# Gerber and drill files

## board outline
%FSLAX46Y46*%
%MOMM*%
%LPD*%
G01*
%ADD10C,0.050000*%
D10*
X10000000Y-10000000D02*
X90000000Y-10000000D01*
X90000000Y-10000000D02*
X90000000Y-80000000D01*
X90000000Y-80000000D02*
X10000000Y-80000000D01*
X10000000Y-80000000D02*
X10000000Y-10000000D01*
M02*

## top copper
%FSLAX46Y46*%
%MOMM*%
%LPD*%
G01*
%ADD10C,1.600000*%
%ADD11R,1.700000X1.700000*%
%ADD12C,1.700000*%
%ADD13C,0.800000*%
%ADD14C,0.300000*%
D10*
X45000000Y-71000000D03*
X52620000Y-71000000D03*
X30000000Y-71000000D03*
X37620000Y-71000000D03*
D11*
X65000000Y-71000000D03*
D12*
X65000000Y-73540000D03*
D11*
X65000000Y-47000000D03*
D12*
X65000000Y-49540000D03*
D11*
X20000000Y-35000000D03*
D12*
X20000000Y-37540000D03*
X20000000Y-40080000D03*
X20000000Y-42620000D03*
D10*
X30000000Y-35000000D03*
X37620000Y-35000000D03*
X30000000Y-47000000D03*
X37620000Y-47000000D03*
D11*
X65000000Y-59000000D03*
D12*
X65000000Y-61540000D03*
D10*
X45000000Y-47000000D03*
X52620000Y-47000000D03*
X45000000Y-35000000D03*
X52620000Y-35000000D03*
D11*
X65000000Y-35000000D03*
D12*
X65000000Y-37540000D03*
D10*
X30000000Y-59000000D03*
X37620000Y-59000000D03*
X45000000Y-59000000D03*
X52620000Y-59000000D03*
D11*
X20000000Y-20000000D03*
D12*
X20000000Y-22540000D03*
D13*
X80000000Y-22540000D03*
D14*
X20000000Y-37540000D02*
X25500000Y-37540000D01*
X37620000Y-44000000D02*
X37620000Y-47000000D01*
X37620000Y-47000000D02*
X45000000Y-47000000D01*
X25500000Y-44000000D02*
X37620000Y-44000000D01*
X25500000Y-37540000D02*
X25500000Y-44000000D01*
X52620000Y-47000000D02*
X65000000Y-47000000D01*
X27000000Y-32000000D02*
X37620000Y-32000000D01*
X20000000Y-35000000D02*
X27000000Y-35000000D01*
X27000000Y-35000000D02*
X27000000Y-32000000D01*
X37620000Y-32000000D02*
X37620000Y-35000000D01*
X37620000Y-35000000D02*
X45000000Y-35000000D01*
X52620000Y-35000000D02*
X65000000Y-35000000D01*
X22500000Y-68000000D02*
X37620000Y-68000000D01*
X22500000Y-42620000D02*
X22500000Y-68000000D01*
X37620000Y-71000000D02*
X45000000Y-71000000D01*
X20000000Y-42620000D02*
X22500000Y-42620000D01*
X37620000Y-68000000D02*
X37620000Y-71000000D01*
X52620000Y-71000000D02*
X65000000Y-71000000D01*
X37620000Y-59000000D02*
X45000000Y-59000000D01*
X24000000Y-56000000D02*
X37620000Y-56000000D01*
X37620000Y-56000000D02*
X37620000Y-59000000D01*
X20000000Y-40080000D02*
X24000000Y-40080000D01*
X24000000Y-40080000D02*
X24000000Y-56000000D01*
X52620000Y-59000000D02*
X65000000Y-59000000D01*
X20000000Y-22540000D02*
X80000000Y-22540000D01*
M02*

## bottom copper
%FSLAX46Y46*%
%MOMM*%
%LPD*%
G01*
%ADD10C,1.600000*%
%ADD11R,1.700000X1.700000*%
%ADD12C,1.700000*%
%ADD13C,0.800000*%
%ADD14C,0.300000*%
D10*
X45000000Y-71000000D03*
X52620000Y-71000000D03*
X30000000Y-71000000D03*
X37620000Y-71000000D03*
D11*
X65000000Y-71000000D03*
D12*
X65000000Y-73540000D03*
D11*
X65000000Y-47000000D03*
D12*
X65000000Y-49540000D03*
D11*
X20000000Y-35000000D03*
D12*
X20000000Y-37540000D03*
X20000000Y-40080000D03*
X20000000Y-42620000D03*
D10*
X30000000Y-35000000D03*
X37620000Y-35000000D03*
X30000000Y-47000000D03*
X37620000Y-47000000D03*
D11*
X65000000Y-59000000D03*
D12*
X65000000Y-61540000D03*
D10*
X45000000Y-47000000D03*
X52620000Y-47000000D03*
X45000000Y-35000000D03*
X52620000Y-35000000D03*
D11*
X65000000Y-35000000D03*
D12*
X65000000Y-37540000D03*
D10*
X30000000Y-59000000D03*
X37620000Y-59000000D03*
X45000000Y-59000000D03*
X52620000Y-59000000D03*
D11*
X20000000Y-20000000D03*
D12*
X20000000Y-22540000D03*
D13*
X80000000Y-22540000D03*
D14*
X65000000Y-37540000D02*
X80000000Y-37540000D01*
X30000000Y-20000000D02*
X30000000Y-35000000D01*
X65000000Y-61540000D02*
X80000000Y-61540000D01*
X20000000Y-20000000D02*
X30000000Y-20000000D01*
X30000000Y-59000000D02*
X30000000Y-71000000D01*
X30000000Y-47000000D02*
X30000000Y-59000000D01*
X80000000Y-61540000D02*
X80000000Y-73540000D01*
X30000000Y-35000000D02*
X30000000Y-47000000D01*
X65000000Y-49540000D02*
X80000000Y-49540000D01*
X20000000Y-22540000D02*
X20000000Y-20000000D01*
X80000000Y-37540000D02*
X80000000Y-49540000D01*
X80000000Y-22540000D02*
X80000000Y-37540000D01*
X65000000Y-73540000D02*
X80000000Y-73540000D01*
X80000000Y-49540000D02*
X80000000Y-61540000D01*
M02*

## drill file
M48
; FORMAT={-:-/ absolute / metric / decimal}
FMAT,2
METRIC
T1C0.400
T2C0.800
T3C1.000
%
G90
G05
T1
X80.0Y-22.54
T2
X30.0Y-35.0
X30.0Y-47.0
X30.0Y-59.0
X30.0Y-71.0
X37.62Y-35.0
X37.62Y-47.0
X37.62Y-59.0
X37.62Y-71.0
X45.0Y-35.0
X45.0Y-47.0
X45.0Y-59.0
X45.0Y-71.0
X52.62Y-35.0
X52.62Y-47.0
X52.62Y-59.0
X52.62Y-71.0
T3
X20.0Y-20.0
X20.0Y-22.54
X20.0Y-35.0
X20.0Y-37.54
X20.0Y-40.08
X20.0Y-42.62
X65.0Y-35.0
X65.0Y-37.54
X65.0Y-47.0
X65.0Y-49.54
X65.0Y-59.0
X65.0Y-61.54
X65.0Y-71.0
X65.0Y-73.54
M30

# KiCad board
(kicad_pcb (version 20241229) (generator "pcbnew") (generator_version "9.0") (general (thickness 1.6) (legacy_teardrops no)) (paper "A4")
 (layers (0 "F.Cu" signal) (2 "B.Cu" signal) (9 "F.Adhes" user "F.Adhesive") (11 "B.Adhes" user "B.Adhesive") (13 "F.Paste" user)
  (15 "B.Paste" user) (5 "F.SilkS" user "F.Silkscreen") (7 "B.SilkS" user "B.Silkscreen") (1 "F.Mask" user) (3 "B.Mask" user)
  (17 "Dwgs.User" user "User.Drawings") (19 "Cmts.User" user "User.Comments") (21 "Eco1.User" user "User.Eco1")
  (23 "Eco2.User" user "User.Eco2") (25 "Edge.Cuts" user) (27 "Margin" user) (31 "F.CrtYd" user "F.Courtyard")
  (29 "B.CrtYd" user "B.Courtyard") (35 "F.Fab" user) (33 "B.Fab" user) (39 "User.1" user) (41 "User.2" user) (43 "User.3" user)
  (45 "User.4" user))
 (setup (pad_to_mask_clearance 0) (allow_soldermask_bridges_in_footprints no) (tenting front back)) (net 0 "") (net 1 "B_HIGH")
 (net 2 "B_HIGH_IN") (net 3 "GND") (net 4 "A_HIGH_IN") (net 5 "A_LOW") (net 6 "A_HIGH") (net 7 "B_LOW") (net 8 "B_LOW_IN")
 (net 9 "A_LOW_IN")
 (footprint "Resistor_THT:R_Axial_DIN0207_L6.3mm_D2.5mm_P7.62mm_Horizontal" (layer "F.Cu") (at 45 71)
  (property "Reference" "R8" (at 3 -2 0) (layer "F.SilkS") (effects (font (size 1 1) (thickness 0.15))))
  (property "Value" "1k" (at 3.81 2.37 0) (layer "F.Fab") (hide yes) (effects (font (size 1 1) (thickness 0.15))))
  (pad "1" thru_hole circle (at 0 0) (size 1.6 1.6) (drill 0.8) (layers "*.Cu" "*.Mask") (remove_unused_layers no) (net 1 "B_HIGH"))
  (pad "2" thru_hole circle (at 7.62 0) (size 1.6 1.6) (drill 0.8) (layers "*.Cu" "*.Mask") (remove_unused_layers no) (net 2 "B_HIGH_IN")))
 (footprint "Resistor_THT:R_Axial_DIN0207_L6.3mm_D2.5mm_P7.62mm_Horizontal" (layer "F.Cu") (at 30 71)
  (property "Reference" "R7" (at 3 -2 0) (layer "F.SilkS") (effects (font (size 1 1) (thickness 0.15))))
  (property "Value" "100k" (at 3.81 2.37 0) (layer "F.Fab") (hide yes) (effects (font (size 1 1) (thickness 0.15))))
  (pad "1" thru_hole circle (at 0 0) (size 1.6 1.6) (drill 0.8) (layers "*.Cu" "*.Mask") (remove_unused_layers no) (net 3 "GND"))
  (pad "2" thru_hole circle (at 7.62 0) (size 1.6 1.6) (drill 0.8) (layers "*.Cu" "*.Mask") (remove_unused_layers no) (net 1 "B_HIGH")))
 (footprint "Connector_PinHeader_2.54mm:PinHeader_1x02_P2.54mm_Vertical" (layer "F.Cu") (at 65 71)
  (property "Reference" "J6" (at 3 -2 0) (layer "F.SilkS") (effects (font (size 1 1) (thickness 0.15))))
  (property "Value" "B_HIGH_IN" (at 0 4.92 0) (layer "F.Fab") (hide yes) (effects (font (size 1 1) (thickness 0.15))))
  (pad "1" thru_hole rect (at 0 0) (size 1.7 1.7) (drill 1) (layers "*.Cu" "*.Mask") (remove_unused_layers no) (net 2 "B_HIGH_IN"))
  (pad "2" thru_hole circle (at 0 2.54) (size 1.7 1.7) (drill 1) (layers "*.Cu" "*.Mask") (remove_unused_layers no) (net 3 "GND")))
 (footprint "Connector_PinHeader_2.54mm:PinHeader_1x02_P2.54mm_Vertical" (layer "F.Cu") (at 65 47)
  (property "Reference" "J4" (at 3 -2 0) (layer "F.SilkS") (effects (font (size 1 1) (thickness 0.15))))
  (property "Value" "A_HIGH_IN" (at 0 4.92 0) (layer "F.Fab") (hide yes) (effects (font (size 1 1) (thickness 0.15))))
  (pad "1" thru_hole rect (at 0 0) (size 1.7 1.7) (drill 1) (layers "*.Cu" "*.Mask") (remove_unused_layers no) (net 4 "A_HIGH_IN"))
  (pad "2" thru_hole circle (at 0 2.54) (size 1.7 1.7) (drill 1) (layers "*.Cu" "*.Mask") (remove_unused_layers no) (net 3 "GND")))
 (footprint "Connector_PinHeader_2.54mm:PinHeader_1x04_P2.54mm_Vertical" (layer "F.Cu") (at 20 35)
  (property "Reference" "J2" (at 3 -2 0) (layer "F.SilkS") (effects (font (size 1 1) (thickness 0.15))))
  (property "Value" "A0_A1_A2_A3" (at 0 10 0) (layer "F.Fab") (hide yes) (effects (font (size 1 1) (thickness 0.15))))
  (pad "1" thru_hole rect (at 0 0) (size 1.7 1.7) (drill 1) (layers "*.Cu" "*.Mask") (remove_unused_layers no) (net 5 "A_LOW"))
  (pad "2" thru_hole circle (at 0 2.54) (size 1.7 1.7) (drill 1) (layers "*.Cu" "*.Mask") (remove_unused_layers no) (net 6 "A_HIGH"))
  (pad "3" thru_hole circle (at 0 5.08) (size 1.7 1.7) (drill 1) (layers "*.Cu" "*.Mask") (remove_unused_layers no) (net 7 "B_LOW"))
  (pad "4" thru_hole circle (at 0 7.62) (size 1.7 1.7) (drill 1) (layers "*.Cu" "*.Mask") (remove_unused_layers no) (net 1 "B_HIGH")))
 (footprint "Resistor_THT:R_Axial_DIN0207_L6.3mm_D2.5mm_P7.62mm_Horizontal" (layer "F.Cu") (at 30 35)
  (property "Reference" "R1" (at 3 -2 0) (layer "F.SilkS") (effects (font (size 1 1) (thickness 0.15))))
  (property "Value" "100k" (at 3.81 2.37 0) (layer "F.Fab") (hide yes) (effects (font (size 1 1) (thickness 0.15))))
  (pad "1" thru_hole circle (at 0 0) (size 1.6 1.6) (drill 0.8) (layers "*.Cu" "*.Mask") (remove_unused_layers no) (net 3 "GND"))
  (pad "2" thru_hole circle (at 7.62 0) (size 1.6 1.6) (drill 0.8) (layers "*.Cu" "*.Mask") (remove_unused_layers no) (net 5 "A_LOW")))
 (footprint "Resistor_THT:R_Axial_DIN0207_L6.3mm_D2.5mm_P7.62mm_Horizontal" (layer "F.Cu") (at 30 47)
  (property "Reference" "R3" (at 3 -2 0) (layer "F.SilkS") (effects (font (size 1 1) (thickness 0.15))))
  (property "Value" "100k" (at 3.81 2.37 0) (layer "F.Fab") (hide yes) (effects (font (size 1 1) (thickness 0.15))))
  (pad "1" thru_hole circle (at 0 0) (size 1.6 1.6) (drill 0.8) (layers "*.Cu" "*.Mask") (remove_unused_layers no) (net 3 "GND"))
  (pad "2" thru_hole circle (at 7.62 0) (size 1.6 1.6) (drill 0.8) (layers "*.Cu" "*.Mask") (remove_unused_layers no) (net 6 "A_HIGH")))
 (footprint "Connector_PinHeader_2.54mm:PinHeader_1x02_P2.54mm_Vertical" (layer "F.Cu") (at 65 59)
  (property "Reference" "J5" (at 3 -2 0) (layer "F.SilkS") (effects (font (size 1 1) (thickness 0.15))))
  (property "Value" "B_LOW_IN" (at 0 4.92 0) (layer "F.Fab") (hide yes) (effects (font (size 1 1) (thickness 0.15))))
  (pad "1" thru_hole rect (at 0 0) (size 1.7 1.7) (drill 1) (layers "*.Cu" "*.Mask") (remove_unused_layers no) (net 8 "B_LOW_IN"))
  (pad "2" thru_hole circle (at 0 2.54) (size 1.7 1.7) (drill 1) (layers "*.Cu" "*.Mask") (remove_unused_layers no) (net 3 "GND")))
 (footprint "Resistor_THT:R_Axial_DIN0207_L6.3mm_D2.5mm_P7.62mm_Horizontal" (layer "F.Cu") (at 45 47)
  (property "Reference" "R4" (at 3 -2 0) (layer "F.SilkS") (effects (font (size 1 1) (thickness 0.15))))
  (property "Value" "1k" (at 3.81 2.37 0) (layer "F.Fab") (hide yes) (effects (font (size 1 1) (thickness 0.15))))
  (pad "1" thru_hole circle (at 0 0) (size 1.6 1.6) (drill 0.8) (layers "*.Cu" "*.Mask") (remove_unused_layers no) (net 6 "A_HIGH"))
  (pad "2" thru_hole circle (at 7.62 0) (size 1.6 1.6) (drill 0.8) (layers "*.Cu" "*.Mask") (remove_unused_layers no) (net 4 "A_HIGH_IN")))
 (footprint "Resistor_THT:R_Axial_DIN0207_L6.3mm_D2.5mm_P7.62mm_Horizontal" (layer "F.Cu") (at 45 35)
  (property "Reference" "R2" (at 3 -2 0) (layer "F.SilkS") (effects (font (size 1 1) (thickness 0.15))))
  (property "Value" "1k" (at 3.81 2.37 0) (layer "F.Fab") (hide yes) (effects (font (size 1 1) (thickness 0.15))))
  (pad "1" thru_hole circle (at 0 0) (size 1.6 1.6) (drill 0.8) (layers "*.Cu" "*.Mask") (remove_unused_layers no) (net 5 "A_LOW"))
  (pad "2" thru_hole circle (at 7.62 0) (size 1.6 1.6) (drill 0.8) (layers "*.Cu" "*.Mask") (remove_unused_layers no) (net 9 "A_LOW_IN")))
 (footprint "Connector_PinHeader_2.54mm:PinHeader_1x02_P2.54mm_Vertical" (layer "F.Cu") (at 65 35)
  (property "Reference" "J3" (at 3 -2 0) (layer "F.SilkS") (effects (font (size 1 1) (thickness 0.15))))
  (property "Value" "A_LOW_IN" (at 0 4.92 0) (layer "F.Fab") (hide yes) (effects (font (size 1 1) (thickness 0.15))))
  (pad "1" thru_hole rect (at 0 0) (size 1.7 1.7) (drill 1) (layers "*.Cu" "*.Mask") (remove_unused_layers no) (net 9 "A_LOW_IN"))
  (pad "2" thru_hole circle (at 0 2.54) (size 1.7 1.7) (drill 1) (layers "*.Cu" "*.Mask") (remove_unused_layers no) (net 3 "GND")))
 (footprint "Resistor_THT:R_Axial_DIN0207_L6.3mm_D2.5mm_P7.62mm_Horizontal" (layer "F.Cu") (at 30 59)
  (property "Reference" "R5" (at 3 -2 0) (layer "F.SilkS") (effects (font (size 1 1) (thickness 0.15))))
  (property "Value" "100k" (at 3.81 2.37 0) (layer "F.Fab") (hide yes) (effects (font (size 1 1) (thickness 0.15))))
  (pad "1" thru_hole circle (at 0 0) (size 1.6 1.6) (drill 0.8) (layers "*.Cu" "*.Mask") (remove_unused_layers no) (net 3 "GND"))
  (pad "2" thru_hole circle (at 7.62 0) (size 1.6 1.6) (drill 0.8) (layers "*.Cu" "*.Mask") (remove_unused_layers no) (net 7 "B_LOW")))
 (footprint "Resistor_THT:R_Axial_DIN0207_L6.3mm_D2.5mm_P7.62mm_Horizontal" (layer "F.Cu") (at 45 59)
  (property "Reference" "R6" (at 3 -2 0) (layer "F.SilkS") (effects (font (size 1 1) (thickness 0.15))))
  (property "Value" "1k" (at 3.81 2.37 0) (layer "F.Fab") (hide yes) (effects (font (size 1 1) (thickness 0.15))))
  (pad "1" thru_hole circle (at 0 0) (size 1.6 1.6) (drill 0.8) (layers "*.Cu" "*.Mask") (remove_unused_layers no) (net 7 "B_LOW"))
  (pad "2" thru_hole circle (at 7.62 0) (size 1.6 1.6) (drill 0.8) (layers "*.Cu" "*.Mask") (remove_unused_layers no) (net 8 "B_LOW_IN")))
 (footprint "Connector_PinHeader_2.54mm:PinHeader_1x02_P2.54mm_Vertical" (layer "F.Cu") (at 20 20)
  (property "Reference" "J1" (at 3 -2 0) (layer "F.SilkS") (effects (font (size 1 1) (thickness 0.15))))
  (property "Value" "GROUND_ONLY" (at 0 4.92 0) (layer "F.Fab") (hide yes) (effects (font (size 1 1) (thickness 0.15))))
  (pad "1" thru_hole rect (at 0 0) (size 1.7 1.7) (drill 1) (layers "*.Cu" "*.Mask") (remove_unused_layers no) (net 3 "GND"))
  (pad "2" thru_hole circle (at 0 2.54) (size 1.7 1.7) (drill 1) (layers "*.Cu" "*.Mask") (remove_unused_layers no) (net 3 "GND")))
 (gr_line (start 10 10) (end 90 10) (stroke (width 0.05) (type default)) (layer "Edge.Cuts"))
 (gr_line (start 90 10) (end 90 80) (stroke (width 0.05) (type default)) (layer "Edge.Cuts"))
 (gr_line (start 90 80) (end 10 80) (stroke (width 0.05) (type default)) (layer "Edge.Cuts"))
 (gr_line (start 10 80) (end 10 10) (stroke (width 0.05) (type default)) (layer "Edge.Cuts"))
 (segment (start 20 37.54) (end 25.5 37.54) (width 0.3) (layer "F.Cu") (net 6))
 (segment (start 37.62 44) (end 37.62 47) (width 0.3) (layer "F.Cu") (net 6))
 (segment (start 37.62 47) (end 45 47) (width 0.3) (layer "F.Cu") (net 6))
 (segment (start 25.5 44) (end 37.62 44) (width 0.3) (layer "F.Cu") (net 6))
 (segment (start 25.5 37.54) (end 25.5 44) (width 0.3) (layer "F.Cu") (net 6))
 (segment (start 52.62 47) (end 65 47) (width 0.3) (layer "F.Cu") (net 4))
 (segment (start 27 32) (end 37.62 32) (width 0.3) (layer "F.Cu") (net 5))
 (segment (start 20 35) (end 27 35) (width 0.3) (layer "F.Cu") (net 5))
 (segment (start 27 35) (end 27 32) (width 0.3) (layer "F.Cu") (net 5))
 (segment (start 37.62 32) (end 37.62 35) (width 0.3) (layer "F.Cu") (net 5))
 (segment (start 37.62 35) (end 45 35) (width 0.3) (layer "F.Cu") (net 5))
 (segment (start 52.62 35) (end 65 35) (width 0.3) (layer "F.Cu") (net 9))
 (segment (start 22.5 68) (end 37.62 68) (width 0.3) (layer "F.Cu") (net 1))
 (segment (start 22.5 42.62) (end 22.5 68) (width 0.3) (layer "F.Cu") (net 1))
 (segment (start 37.62 71) (end 45 71) (width 0.3) (layer "F.Cu") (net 1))
 (segment (start 20 42.62) (end 22.5 42.62) (width 0.3) (layer "F.Cu") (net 1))
 (segment (start 37.62 68) (end 37.62 71) (width 0.3) (layer "F.Cu") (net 1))
 (segment (start 52.62 71) (end 65 71) (width 0.3) (layer "F.Cu") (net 2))
 (segment (start 37.62 59) (end 45 59) (width 0.3) (layer "F.Cu") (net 7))
 (segment (start 24 56) (end 37.62 56) (width 0.3) (layer "F.Cu") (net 7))
 (segment (start 37.62 56) (end 37.62 59) (width 0.3) (layer "F.Cu") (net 7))
 (segment (start 20 40.08) (end 24 40.08) (width 0.3) (layer "F.Cu") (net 7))
 (segment (start 24 40.08) (end 24 56) (width 0.3) (layer "F.Cu") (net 7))
 (segment (start 52.62 59) (end 65 59) (width 0.3) (layer "F.Cu") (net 8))
 (segment (start 20 22.54) (end 80 22.54) (width 0.3) (layer "F.Cu") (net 3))
 (via (at 80 22.54) (size 0.8) (drill 0.4) (layers "F.Cu" "B.Cu") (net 3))
 (segment (start 65 37.54) (end 80 37.54) (width 0.3) (layer "B.Cu") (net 3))
 (segment (start 30 20) (end 30 35) (width 0.3) (layer "B.Cu") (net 3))
 (segment (start 65 61.54) (end 80 61.54) (width 0.3) (layer "B.Cu") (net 3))
 (segment (start 20 20) (end 30 20) (width 0.3) (layer "B.Cu") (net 3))
 (segment (start 30 59) (end 30 71) (width 0.3) (layer "B.Cu") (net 3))
 (segment (start 30 47) (end 30 59) (width 0.3) (layer "B.Cu") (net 3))
 (segment (start 80 61.54) (end 80 73.54) (width 0.3) (layer "B.Cu") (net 3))
 (segment (start 30 35) (end 30 47) (width 0.3) (layer "B.Cu") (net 3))
 (segment (start 65 49.54) (end 80 49.54) (width 0.3) (layer "B.Cu") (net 3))
 (segment (start 20 22.54) (end 20 20) (width 0.3) (layer "B.Cu") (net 3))
 (segment (start 80 37.54) (end 80 49.54) (width 0.3) (layer "B.Cu") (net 3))
 (segment (start 80 22.54) (end 80 37.54) (width 0.3) (layer "B.Cu") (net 3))
 (segment (start 65 73.54) (end 80 73.54) (width 0.3) (layer "B.Cu") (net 3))
 (segment (start 80 49.54) (end 80 61.54) (width 0.3) (layer "B.Cu") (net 3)))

